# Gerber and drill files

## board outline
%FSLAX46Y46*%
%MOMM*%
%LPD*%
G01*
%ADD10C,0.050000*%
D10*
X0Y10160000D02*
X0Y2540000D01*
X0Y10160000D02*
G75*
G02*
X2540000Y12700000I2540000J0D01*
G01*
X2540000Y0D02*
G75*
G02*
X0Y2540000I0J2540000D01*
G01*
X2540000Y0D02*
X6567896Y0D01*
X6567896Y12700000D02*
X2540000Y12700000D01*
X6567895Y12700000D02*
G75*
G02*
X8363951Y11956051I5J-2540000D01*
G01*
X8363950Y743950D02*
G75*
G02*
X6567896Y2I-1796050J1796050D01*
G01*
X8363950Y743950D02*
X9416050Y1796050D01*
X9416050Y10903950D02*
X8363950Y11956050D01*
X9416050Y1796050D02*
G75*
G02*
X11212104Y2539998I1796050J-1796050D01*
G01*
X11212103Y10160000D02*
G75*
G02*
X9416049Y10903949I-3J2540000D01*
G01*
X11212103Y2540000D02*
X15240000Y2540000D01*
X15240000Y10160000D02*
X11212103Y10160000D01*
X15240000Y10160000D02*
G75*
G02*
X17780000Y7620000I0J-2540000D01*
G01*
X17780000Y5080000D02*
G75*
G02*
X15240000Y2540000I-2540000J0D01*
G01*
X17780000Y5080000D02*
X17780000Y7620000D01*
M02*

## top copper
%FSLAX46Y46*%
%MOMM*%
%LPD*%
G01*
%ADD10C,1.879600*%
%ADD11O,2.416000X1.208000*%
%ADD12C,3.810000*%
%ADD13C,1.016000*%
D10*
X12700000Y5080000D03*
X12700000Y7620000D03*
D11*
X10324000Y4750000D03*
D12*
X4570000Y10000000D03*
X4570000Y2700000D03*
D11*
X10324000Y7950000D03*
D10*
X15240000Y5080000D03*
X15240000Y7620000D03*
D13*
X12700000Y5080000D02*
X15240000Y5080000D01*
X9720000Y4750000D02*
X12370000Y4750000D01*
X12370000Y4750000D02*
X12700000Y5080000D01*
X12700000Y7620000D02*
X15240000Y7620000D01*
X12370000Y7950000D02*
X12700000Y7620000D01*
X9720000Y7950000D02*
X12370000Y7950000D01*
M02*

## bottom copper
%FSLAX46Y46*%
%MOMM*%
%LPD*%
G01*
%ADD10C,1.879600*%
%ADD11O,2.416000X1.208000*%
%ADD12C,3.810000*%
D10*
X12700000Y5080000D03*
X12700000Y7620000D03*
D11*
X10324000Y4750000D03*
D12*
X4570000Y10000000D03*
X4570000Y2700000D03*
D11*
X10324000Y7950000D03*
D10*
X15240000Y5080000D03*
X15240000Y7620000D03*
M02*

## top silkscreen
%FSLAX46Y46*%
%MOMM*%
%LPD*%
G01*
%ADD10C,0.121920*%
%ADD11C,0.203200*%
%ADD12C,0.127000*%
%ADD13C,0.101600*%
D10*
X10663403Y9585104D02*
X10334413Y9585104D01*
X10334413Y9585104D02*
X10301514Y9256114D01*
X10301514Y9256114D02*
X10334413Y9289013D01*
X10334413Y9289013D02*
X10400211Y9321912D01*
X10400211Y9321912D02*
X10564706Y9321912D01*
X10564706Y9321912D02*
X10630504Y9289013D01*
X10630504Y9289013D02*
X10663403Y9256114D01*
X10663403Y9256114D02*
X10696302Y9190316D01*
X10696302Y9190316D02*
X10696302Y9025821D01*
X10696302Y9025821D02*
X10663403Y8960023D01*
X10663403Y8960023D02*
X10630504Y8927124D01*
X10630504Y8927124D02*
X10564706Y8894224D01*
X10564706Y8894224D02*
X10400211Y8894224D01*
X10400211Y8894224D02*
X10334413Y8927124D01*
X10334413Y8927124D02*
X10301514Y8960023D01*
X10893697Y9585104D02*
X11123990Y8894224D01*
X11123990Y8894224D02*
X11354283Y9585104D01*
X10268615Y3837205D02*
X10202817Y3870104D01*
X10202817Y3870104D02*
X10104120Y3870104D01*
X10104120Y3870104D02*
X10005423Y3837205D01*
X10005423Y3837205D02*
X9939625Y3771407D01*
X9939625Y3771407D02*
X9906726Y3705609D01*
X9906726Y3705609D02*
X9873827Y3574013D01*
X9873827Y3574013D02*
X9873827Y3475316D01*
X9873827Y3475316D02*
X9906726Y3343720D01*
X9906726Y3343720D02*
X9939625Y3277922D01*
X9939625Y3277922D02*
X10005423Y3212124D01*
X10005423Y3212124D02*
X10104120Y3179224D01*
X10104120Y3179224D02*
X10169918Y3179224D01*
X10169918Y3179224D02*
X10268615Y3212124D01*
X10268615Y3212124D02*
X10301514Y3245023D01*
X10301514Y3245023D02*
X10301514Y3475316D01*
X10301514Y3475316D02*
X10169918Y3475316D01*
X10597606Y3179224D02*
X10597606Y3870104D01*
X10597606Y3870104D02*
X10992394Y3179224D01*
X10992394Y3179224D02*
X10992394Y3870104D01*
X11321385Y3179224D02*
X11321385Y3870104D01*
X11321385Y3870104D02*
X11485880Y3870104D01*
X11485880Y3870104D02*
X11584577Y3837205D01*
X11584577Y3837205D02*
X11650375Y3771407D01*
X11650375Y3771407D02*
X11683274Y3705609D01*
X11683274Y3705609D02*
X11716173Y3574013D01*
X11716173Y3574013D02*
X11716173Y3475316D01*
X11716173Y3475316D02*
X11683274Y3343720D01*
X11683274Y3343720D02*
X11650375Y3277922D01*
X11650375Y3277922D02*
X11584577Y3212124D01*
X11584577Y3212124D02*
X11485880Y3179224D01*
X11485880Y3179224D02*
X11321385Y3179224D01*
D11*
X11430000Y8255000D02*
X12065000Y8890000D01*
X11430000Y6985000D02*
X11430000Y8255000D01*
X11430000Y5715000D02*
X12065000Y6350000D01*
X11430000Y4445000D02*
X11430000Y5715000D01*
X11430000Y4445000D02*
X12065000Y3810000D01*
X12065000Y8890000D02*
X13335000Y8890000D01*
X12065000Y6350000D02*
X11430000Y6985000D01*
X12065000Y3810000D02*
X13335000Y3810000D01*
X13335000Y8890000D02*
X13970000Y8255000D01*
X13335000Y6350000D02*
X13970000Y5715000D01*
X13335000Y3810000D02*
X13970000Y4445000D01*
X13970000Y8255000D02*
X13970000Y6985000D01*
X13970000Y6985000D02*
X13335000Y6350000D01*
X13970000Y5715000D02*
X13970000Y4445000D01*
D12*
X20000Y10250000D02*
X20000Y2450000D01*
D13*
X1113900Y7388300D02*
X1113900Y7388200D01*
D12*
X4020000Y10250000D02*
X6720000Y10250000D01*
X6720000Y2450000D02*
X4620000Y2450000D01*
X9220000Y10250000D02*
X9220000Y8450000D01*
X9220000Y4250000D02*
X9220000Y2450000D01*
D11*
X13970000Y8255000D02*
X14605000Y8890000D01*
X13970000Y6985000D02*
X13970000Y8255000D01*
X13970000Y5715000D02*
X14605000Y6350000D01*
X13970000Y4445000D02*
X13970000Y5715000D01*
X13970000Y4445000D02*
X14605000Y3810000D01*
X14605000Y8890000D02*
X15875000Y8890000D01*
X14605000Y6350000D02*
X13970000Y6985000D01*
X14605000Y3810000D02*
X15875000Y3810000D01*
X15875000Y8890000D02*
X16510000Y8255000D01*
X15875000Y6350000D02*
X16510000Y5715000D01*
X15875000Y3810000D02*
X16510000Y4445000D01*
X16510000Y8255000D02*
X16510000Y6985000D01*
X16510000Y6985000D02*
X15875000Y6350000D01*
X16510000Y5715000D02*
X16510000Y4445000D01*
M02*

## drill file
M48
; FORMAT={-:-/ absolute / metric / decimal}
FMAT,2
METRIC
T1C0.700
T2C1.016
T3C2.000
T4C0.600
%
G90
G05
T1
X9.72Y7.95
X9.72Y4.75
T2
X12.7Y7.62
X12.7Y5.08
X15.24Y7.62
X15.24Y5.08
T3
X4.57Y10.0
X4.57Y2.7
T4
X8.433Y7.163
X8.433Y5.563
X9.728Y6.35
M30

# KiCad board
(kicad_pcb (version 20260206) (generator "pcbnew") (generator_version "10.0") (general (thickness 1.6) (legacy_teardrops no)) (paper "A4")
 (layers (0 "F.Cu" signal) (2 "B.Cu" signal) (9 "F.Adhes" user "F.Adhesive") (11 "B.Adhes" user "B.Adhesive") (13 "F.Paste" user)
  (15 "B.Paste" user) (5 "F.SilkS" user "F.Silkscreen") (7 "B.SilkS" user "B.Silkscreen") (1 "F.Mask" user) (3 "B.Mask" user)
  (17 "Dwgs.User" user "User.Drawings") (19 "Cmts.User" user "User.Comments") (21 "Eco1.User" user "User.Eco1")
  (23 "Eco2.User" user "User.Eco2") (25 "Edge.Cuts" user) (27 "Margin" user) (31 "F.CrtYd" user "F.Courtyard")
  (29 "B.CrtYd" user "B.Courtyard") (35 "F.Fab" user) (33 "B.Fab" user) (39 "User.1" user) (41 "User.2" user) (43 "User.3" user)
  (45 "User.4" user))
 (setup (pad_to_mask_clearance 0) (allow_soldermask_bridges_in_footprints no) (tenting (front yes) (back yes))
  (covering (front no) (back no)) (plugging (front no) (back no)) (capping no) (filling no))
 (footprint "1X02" (layer "F.Cu") (at 12.7 -5.08 90)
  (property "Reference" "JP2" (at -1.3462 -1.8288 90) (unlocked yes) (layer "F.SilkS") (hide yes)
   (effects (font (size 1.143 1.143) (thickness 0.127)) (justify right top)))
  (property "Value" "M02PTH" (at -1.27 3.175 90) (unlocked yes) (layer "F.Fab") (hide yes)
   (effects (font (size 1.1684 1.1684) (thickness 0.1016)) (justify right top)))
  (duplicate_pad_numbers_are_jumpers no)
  (fp_line (start 3.175 -1.27) (end 3.81 -0.635) (stroke (width 0.2032) (type solid)) (layer "F.SilkS"))
  (fp_line (start 1.905 -1.27) (end 3.175 -1.27) (stroke (width 0.2032) (type solid)) (layer "F.SilkS"))
  (fp_line (start 0.635 -1.27) (end 1.27 -0.635) (stroke (width 0.2032) (type solid)) (layer "F.SilkS"))
  (fp_line (start -0.635 -1.27) (end 0.635 -1.27) (stroke (width 0.2032) (type solid)) (layer "F.SilkS"))
  (fp_line (start -0.635 -1.27) (end -1.27 -0.635) (stroke (width 0.2032) (type solid)) (layer "F.SilkS"))
  (fp_line (start 3.81 -0.635) (end 3.81 0.635) (stroke (width 0.2032) (type solid)) (layer "F.SilkS"))
  (fp_line (start 1.27 -0.635) (end 1.905 -1.27) (stroke (width 0.2032) (type solid)) (layer "F.SilkS"))
  (fp_line (start -1.27 -0.635) (end -1.27 0.635) (stroke (width 0.2032) (type solid)) (layer "F.SilkS"))
  (fp_line (start 3.81 0.635) (end 3.175 1.27) (stroke (width 0.2032) (type solid)) (layer "F.SilkS"))
  (fp_line (start 1.27 0.635) (end 0.635 1.27) (stroke (width 0.2032) (type solid)) (layer "F.SilkS"))
  (fp_line (start -1.27 0.635) (end -0.635 1.27) (stroke (width 0.2032) (type solid)) (layer "F.SilkS"))
  (fp_line (start 3.175 1.27) (end 1.905 1.27) (stroke (width 0.2032) (type solid)) (layer "F.SilkS"))
  (fp_line (start 1.905 1.27) (end 1.27 0.635) (stroke (width 0.2032) (type solid)) (layer "F.SilkS"))
  (fp_line (start 0.635 1.27) (end -0.635 1.27) (stroke (width 0.2032) (type solid)) (layer "F.SilkS"))
  (pad "1" thru_hole circle (at 0 0 180) (size 1.8796 1.8796) (drill 1.016) (layers "*.Cu" "*.Mask") (remove_unused_layers no) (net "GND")
   (solder_mask_margin 0.1016) (thermal_bridge_angle 0))
  (pad "2" thru_hole circle (at 2.54 0 180) (size 1.8796 1.8796) (drill 1.016) (layers "*.Cu" "*.Mask") (remove_unused_layers no) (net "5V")
   (solder_mask_margin 0.1016) (thermal_bridge_angle 0)))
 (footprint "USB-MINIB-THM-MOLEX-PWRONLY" (layer "F.Cu") (at 5.08 -6.35 -90)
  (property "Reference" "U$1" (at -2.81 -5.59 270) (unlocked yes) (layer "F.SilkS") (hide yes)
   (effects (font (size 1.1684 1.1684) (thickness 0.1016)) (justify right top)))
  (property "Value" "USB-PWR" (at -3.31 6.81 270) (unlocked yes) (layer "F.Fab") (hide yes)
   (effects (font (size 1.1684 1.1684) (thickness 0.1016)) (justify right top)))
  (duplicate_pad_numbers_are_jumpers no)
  (fp_line (start -3.9 5.06) (end 3.9 5.06) (stroke (width 0.127) (type solid)) (layer "F.SilkS"))
  (fp_line (start -1.0383 3.9661) (end -1.0382 3.9661) (stroke (width 0.1016) (type solid)) (layer "F.SilkS"))
  (fp_line (start -3.9 1.06) (end -3.9 -1.64) (stroke (width 0.127) (type solid)) (layer "F.SilkS"))
  (fp_line (start 3.9 -1.64) (end 3.9 0.46) (stroke (width 0.127) (type solid)) (layer "F.SilkS"))
  (fp_line (start -3.9 -4.14) (end -2.1 -4.14) (stroke (width 0.127) (type solid)) (layer "F.SilkS"))
  (fp_line (start 2.1 -4.14) (end 3.9 -4.14) (stroke (width 0.127) (type solid)) (layer "F.SilkS"))
  (pad "" np_thru_hole circle (at -0.8128 -3.3528 270) (size 0.6 0.6) (drill 0.6) (layers "*.Cu" "*.Mask"))
  (pad "" np_thru_hole circle (at 0 -4.6482 270) (size 0.6 0.6) (drill 0.6) (layers "*.Cu" "*.Mask"))
  (pad "" np_thru_hole circle (at 0.7874 -3.3528 270) (size 0.6 0.6) (drill 0.6) (layers "*.Cu" "*.Mask"))
  (pad "GND" thru_hole oval (at 1.6 -4.64) (size 2.416 1.208) (drill 0.7 (offset 0.604 0)) (layers "*.Cu" "*.Mask")
   (remove_unused_layers no) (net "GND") (solder_mask_margin 0.1016) (thermal_bridge_angle 0))
  (pad "GND1" thru_hole circle (at -3.65 0.51 270) (size 3.81 3.81) (drill 2) (layers "*.Cu" "*.Mask") (remove_unused_layers no)
   (solder_mask_margin 0.1016) (thermal_bridge_angle 0))
  (pad "GND4" thru_hole circle (at 3.65 0.51 270) (size 3.81 3.81) (drill 2) (layers "*.Cu" "*.Mask") (remove_unused_layers no)
   (solder_mask_margin 0.1016) (thermal_bridge_angle 0))
  (pad "VBUS" thru_hole oval (at -1.6 -4.64) (size 2.416 1.208) (drill 0.7 (offset 0.604 0)) (layers "*.Cu" "*.Mask")
   (remove_unused_layers no) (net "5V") (solder_mask_margin 0.1016) (thermal_bridge_angle 0)))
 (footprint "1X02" (layer "F.Cu") (at 15.24 -5.08 90)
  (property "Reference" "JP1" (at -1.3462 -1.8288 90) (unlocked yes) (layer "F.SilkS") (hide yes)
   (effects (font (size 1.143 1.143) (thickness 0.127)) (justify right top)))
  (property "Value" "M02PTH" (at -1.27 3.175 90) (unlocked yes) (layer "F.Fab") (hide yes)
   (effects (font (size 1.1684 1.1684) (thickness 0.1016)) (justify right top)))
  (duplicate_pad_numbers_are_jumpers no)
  (fp_line (start 3.175 -1.27) (end 3.81 -0.635) (stroke (width 0.2032) (type solid)) (layer "F.SilkS"))
  (fp_line (start 1.905 -1.27) (end 3.175 -1.27) (stroke (width 0.2032) (type solid)) (layer "F.SilkS"))
  (fp_line (start 0.635 -1.27) (end 1.27 -0.635) (stroke (width 0.2032) (type solid)) (layer "F.SilkS"))
  (fp_line (start -0.635 -1.27) (end 0.635 -1.27) (stroke (width 0.2032) (type solid)) (layer "F.SilkS"))
  (fp_line (start -0.635 -1.27) (end -1.27 -0.635) (stroke (width 0.2032) (type solid)) (layer "F.SilkS"))
  (fp_line (start 3.81 -0.635) (end 3.81 0.635) (stroke (width 0.2032) (type solid)) (layer "F.SilkS"))
  (fp_line (start 1.27 -0.635) (end 1.905 -1.27) (stroke (width 0.2032) (type solid)) (layer "F.SilkS"))
  (fp_line (start -1.27 -0.635) (end -1.27 0.635) (stroke (width 0.2032) (type solid)) (layer "F.SilkS"))
  (fp_line (start 3.81 0.635) (end 3.175 1.27) (stroke (width 0.2032) (type solid)) (layer "F.SilkS"))
  (fp_line (start 1.27 0.635) (end 0.635 1.27) (stroke (width 0.2032) (type solid)) (layer "F.SilkS"))
  (fp_line (start -1.27 0.635) (end -0.635 1.27) (stroke (width 0.2032) (type solid)) (layer "F.SilkS"))
  (fp_line (start 3.175 1.27) (end 1.905 1.27) (stroke (width 0.2032) (type solid)) (layer "F.SilkS"))
  (fp_line (start 1.905 1.27) (end 1.27 0.635) (stroke (width 0.2032) (type solid)) (layer "F.SilkS"))
  (fp_line (start 0.635 1.27) (end -0.635 1.27) (stroke (width 0.2032) (type solid)) (layer "F.SilkS"))
  (pad "1" thru_hole circle (at 0 0 180) (size 1.8796 1.8796) (drill 1.016) (layers "*.Cu" "*.Mask") (remove_unused_layers no) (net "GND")
   (solder_mask_margin 0.1016) (thermal_bridge_angle 0))
  (pad "2" thru_hole circle (at 2.54 0 180) (size 1.8796 1.8796) (drill 1.016) (layers "*.Cu" "*.Mask") (remove_unused_layers no) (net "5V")
   (solder_mask_margin 0.1016) (thermal_bridge_angle 0)))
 (gr_line (start 0 -10.16) (end 0 -2.54) (stroke (width 0.05) (type solid)) (layer "Edge.Cuts"))
 (gr_arc (start 0 -10.16) (mid 0.743949 -11.956051) (end 2.54 -12.7) (stroke (width 0.05) (type solid)) (layer "Edge.Cuts"))
 (gr_arc (start 2.54 0) (mid 0.743949 -0.743949) (end 0 -2.54) (stroke (width 0.05) (type solid)) (layer "Edge.Cuts"))
 (gr_line (start 2.54 0) (end 6.567896 0) (stroke (width 0.05) (type solid)) (layer "Edge.Cuts"))
 (gr_line (start 6.567896 -12.7) (end 2.54 -12.7) (stroke (width 0.05) (type solid)) (layer "Edge.Cuts"))
 (gr_arc (start 6.567895 -12.7) (mid 7.539913 -12.506654) (end 8.36395 -11.95605) (stroke (width 0.05) (type solid)) (layer "Edge.Cuts"))
 (gr_arc (start 8.36395 -0.74395) (mid 7.539914 -0.193346) (end 6.567896 0) (stroke (width 0.05) (type solid)) (layer "Edge.Cuts"))
 (gr_line (start 8.36395 -0.74395) (end 9.41605 -1.79605) (stroke (width 0.05) (type solid)) (layer "Edge.Cuts"))
 (gr_line (start 9.41605 -10.90395) (end 8.36395 -11.95605) (stroke (width 0.05) (type solid)) (layer "Edge.Cuts"))
 (gr_arc (start 9.41605 -1.79605) (mid 10.240086 -2.346654) (end 11.212104 -2.54) (stroke (width 0.05) (type solid)) (layer "Edge.Cuts"))
 (gr_arc (start 11.212103 -10.16) (mid 10.240086 -10.353346) (end 9.41605 -10.90395) (stroke (width 0.05) (type solid)) (layer "Edge.Cuts"))
 (gr_line (start 11.212103 -2.54) (end 15.24 -2.54) (stroke (width 0.05) (type solid)) (layer "Edge.Cuts"))
 (gr_line (start 15.24 -10.16) (end 11.212103 -10.16) (stroke (width 0.05) (type solid)) (layer "Edge.Cuts"))
 (gr_arc (start 15.24 -10.16) (mid 17.036051 -9.416051) (end 17.78 -7.62) (stroke (width 0.05) (type solid)) (layer "Edge.Cuts"))
 (gr_arc (start 17.78 -5.08) (mid 17.036051 -3.283949) (end 15.24 -2.54) (stroke (width 0.05) (type solid)) (layer "Edge.Cuts"))
 (gr_line (start 17.78 -5.08) (end 17.78 -7.62) (stroke (width 0.05) (type solid)) (layer "Edge.Cuts"))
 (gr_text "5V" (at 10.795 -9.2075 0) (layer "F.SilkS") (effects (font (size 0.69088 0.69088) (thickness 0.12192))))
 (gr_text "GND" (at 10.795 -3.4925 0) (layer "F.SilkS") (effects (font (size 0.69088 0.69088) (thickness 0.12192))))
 (segment (start 12.7 -5.08) (end 15.24 -5.08) (width 1.016) (layer "F.Cu") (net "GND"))
 (segment (start 9.72 -4.75) (end 12.37 -4.75) (width 1.016) (layer "F.Cu") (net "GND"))
 (segment (start 12.37 -4.75) (end 12.7 -5.08) (width 1.016) (layer "F.Cu") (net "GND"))
 (segment (start 12.7 -7.62) (end 15.24 -7.62) (width 1.016) (layer "F.Cu") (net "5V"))
 (segment (start 12.37 -7.95) (end 12.7 -7.62) (width 1.016) (layer "F.Cu") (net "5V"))
 (segment (start 9.72 -7.95) (end 12.37 -7.95) (width 1.016) (layer "F.Cu") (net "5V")))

